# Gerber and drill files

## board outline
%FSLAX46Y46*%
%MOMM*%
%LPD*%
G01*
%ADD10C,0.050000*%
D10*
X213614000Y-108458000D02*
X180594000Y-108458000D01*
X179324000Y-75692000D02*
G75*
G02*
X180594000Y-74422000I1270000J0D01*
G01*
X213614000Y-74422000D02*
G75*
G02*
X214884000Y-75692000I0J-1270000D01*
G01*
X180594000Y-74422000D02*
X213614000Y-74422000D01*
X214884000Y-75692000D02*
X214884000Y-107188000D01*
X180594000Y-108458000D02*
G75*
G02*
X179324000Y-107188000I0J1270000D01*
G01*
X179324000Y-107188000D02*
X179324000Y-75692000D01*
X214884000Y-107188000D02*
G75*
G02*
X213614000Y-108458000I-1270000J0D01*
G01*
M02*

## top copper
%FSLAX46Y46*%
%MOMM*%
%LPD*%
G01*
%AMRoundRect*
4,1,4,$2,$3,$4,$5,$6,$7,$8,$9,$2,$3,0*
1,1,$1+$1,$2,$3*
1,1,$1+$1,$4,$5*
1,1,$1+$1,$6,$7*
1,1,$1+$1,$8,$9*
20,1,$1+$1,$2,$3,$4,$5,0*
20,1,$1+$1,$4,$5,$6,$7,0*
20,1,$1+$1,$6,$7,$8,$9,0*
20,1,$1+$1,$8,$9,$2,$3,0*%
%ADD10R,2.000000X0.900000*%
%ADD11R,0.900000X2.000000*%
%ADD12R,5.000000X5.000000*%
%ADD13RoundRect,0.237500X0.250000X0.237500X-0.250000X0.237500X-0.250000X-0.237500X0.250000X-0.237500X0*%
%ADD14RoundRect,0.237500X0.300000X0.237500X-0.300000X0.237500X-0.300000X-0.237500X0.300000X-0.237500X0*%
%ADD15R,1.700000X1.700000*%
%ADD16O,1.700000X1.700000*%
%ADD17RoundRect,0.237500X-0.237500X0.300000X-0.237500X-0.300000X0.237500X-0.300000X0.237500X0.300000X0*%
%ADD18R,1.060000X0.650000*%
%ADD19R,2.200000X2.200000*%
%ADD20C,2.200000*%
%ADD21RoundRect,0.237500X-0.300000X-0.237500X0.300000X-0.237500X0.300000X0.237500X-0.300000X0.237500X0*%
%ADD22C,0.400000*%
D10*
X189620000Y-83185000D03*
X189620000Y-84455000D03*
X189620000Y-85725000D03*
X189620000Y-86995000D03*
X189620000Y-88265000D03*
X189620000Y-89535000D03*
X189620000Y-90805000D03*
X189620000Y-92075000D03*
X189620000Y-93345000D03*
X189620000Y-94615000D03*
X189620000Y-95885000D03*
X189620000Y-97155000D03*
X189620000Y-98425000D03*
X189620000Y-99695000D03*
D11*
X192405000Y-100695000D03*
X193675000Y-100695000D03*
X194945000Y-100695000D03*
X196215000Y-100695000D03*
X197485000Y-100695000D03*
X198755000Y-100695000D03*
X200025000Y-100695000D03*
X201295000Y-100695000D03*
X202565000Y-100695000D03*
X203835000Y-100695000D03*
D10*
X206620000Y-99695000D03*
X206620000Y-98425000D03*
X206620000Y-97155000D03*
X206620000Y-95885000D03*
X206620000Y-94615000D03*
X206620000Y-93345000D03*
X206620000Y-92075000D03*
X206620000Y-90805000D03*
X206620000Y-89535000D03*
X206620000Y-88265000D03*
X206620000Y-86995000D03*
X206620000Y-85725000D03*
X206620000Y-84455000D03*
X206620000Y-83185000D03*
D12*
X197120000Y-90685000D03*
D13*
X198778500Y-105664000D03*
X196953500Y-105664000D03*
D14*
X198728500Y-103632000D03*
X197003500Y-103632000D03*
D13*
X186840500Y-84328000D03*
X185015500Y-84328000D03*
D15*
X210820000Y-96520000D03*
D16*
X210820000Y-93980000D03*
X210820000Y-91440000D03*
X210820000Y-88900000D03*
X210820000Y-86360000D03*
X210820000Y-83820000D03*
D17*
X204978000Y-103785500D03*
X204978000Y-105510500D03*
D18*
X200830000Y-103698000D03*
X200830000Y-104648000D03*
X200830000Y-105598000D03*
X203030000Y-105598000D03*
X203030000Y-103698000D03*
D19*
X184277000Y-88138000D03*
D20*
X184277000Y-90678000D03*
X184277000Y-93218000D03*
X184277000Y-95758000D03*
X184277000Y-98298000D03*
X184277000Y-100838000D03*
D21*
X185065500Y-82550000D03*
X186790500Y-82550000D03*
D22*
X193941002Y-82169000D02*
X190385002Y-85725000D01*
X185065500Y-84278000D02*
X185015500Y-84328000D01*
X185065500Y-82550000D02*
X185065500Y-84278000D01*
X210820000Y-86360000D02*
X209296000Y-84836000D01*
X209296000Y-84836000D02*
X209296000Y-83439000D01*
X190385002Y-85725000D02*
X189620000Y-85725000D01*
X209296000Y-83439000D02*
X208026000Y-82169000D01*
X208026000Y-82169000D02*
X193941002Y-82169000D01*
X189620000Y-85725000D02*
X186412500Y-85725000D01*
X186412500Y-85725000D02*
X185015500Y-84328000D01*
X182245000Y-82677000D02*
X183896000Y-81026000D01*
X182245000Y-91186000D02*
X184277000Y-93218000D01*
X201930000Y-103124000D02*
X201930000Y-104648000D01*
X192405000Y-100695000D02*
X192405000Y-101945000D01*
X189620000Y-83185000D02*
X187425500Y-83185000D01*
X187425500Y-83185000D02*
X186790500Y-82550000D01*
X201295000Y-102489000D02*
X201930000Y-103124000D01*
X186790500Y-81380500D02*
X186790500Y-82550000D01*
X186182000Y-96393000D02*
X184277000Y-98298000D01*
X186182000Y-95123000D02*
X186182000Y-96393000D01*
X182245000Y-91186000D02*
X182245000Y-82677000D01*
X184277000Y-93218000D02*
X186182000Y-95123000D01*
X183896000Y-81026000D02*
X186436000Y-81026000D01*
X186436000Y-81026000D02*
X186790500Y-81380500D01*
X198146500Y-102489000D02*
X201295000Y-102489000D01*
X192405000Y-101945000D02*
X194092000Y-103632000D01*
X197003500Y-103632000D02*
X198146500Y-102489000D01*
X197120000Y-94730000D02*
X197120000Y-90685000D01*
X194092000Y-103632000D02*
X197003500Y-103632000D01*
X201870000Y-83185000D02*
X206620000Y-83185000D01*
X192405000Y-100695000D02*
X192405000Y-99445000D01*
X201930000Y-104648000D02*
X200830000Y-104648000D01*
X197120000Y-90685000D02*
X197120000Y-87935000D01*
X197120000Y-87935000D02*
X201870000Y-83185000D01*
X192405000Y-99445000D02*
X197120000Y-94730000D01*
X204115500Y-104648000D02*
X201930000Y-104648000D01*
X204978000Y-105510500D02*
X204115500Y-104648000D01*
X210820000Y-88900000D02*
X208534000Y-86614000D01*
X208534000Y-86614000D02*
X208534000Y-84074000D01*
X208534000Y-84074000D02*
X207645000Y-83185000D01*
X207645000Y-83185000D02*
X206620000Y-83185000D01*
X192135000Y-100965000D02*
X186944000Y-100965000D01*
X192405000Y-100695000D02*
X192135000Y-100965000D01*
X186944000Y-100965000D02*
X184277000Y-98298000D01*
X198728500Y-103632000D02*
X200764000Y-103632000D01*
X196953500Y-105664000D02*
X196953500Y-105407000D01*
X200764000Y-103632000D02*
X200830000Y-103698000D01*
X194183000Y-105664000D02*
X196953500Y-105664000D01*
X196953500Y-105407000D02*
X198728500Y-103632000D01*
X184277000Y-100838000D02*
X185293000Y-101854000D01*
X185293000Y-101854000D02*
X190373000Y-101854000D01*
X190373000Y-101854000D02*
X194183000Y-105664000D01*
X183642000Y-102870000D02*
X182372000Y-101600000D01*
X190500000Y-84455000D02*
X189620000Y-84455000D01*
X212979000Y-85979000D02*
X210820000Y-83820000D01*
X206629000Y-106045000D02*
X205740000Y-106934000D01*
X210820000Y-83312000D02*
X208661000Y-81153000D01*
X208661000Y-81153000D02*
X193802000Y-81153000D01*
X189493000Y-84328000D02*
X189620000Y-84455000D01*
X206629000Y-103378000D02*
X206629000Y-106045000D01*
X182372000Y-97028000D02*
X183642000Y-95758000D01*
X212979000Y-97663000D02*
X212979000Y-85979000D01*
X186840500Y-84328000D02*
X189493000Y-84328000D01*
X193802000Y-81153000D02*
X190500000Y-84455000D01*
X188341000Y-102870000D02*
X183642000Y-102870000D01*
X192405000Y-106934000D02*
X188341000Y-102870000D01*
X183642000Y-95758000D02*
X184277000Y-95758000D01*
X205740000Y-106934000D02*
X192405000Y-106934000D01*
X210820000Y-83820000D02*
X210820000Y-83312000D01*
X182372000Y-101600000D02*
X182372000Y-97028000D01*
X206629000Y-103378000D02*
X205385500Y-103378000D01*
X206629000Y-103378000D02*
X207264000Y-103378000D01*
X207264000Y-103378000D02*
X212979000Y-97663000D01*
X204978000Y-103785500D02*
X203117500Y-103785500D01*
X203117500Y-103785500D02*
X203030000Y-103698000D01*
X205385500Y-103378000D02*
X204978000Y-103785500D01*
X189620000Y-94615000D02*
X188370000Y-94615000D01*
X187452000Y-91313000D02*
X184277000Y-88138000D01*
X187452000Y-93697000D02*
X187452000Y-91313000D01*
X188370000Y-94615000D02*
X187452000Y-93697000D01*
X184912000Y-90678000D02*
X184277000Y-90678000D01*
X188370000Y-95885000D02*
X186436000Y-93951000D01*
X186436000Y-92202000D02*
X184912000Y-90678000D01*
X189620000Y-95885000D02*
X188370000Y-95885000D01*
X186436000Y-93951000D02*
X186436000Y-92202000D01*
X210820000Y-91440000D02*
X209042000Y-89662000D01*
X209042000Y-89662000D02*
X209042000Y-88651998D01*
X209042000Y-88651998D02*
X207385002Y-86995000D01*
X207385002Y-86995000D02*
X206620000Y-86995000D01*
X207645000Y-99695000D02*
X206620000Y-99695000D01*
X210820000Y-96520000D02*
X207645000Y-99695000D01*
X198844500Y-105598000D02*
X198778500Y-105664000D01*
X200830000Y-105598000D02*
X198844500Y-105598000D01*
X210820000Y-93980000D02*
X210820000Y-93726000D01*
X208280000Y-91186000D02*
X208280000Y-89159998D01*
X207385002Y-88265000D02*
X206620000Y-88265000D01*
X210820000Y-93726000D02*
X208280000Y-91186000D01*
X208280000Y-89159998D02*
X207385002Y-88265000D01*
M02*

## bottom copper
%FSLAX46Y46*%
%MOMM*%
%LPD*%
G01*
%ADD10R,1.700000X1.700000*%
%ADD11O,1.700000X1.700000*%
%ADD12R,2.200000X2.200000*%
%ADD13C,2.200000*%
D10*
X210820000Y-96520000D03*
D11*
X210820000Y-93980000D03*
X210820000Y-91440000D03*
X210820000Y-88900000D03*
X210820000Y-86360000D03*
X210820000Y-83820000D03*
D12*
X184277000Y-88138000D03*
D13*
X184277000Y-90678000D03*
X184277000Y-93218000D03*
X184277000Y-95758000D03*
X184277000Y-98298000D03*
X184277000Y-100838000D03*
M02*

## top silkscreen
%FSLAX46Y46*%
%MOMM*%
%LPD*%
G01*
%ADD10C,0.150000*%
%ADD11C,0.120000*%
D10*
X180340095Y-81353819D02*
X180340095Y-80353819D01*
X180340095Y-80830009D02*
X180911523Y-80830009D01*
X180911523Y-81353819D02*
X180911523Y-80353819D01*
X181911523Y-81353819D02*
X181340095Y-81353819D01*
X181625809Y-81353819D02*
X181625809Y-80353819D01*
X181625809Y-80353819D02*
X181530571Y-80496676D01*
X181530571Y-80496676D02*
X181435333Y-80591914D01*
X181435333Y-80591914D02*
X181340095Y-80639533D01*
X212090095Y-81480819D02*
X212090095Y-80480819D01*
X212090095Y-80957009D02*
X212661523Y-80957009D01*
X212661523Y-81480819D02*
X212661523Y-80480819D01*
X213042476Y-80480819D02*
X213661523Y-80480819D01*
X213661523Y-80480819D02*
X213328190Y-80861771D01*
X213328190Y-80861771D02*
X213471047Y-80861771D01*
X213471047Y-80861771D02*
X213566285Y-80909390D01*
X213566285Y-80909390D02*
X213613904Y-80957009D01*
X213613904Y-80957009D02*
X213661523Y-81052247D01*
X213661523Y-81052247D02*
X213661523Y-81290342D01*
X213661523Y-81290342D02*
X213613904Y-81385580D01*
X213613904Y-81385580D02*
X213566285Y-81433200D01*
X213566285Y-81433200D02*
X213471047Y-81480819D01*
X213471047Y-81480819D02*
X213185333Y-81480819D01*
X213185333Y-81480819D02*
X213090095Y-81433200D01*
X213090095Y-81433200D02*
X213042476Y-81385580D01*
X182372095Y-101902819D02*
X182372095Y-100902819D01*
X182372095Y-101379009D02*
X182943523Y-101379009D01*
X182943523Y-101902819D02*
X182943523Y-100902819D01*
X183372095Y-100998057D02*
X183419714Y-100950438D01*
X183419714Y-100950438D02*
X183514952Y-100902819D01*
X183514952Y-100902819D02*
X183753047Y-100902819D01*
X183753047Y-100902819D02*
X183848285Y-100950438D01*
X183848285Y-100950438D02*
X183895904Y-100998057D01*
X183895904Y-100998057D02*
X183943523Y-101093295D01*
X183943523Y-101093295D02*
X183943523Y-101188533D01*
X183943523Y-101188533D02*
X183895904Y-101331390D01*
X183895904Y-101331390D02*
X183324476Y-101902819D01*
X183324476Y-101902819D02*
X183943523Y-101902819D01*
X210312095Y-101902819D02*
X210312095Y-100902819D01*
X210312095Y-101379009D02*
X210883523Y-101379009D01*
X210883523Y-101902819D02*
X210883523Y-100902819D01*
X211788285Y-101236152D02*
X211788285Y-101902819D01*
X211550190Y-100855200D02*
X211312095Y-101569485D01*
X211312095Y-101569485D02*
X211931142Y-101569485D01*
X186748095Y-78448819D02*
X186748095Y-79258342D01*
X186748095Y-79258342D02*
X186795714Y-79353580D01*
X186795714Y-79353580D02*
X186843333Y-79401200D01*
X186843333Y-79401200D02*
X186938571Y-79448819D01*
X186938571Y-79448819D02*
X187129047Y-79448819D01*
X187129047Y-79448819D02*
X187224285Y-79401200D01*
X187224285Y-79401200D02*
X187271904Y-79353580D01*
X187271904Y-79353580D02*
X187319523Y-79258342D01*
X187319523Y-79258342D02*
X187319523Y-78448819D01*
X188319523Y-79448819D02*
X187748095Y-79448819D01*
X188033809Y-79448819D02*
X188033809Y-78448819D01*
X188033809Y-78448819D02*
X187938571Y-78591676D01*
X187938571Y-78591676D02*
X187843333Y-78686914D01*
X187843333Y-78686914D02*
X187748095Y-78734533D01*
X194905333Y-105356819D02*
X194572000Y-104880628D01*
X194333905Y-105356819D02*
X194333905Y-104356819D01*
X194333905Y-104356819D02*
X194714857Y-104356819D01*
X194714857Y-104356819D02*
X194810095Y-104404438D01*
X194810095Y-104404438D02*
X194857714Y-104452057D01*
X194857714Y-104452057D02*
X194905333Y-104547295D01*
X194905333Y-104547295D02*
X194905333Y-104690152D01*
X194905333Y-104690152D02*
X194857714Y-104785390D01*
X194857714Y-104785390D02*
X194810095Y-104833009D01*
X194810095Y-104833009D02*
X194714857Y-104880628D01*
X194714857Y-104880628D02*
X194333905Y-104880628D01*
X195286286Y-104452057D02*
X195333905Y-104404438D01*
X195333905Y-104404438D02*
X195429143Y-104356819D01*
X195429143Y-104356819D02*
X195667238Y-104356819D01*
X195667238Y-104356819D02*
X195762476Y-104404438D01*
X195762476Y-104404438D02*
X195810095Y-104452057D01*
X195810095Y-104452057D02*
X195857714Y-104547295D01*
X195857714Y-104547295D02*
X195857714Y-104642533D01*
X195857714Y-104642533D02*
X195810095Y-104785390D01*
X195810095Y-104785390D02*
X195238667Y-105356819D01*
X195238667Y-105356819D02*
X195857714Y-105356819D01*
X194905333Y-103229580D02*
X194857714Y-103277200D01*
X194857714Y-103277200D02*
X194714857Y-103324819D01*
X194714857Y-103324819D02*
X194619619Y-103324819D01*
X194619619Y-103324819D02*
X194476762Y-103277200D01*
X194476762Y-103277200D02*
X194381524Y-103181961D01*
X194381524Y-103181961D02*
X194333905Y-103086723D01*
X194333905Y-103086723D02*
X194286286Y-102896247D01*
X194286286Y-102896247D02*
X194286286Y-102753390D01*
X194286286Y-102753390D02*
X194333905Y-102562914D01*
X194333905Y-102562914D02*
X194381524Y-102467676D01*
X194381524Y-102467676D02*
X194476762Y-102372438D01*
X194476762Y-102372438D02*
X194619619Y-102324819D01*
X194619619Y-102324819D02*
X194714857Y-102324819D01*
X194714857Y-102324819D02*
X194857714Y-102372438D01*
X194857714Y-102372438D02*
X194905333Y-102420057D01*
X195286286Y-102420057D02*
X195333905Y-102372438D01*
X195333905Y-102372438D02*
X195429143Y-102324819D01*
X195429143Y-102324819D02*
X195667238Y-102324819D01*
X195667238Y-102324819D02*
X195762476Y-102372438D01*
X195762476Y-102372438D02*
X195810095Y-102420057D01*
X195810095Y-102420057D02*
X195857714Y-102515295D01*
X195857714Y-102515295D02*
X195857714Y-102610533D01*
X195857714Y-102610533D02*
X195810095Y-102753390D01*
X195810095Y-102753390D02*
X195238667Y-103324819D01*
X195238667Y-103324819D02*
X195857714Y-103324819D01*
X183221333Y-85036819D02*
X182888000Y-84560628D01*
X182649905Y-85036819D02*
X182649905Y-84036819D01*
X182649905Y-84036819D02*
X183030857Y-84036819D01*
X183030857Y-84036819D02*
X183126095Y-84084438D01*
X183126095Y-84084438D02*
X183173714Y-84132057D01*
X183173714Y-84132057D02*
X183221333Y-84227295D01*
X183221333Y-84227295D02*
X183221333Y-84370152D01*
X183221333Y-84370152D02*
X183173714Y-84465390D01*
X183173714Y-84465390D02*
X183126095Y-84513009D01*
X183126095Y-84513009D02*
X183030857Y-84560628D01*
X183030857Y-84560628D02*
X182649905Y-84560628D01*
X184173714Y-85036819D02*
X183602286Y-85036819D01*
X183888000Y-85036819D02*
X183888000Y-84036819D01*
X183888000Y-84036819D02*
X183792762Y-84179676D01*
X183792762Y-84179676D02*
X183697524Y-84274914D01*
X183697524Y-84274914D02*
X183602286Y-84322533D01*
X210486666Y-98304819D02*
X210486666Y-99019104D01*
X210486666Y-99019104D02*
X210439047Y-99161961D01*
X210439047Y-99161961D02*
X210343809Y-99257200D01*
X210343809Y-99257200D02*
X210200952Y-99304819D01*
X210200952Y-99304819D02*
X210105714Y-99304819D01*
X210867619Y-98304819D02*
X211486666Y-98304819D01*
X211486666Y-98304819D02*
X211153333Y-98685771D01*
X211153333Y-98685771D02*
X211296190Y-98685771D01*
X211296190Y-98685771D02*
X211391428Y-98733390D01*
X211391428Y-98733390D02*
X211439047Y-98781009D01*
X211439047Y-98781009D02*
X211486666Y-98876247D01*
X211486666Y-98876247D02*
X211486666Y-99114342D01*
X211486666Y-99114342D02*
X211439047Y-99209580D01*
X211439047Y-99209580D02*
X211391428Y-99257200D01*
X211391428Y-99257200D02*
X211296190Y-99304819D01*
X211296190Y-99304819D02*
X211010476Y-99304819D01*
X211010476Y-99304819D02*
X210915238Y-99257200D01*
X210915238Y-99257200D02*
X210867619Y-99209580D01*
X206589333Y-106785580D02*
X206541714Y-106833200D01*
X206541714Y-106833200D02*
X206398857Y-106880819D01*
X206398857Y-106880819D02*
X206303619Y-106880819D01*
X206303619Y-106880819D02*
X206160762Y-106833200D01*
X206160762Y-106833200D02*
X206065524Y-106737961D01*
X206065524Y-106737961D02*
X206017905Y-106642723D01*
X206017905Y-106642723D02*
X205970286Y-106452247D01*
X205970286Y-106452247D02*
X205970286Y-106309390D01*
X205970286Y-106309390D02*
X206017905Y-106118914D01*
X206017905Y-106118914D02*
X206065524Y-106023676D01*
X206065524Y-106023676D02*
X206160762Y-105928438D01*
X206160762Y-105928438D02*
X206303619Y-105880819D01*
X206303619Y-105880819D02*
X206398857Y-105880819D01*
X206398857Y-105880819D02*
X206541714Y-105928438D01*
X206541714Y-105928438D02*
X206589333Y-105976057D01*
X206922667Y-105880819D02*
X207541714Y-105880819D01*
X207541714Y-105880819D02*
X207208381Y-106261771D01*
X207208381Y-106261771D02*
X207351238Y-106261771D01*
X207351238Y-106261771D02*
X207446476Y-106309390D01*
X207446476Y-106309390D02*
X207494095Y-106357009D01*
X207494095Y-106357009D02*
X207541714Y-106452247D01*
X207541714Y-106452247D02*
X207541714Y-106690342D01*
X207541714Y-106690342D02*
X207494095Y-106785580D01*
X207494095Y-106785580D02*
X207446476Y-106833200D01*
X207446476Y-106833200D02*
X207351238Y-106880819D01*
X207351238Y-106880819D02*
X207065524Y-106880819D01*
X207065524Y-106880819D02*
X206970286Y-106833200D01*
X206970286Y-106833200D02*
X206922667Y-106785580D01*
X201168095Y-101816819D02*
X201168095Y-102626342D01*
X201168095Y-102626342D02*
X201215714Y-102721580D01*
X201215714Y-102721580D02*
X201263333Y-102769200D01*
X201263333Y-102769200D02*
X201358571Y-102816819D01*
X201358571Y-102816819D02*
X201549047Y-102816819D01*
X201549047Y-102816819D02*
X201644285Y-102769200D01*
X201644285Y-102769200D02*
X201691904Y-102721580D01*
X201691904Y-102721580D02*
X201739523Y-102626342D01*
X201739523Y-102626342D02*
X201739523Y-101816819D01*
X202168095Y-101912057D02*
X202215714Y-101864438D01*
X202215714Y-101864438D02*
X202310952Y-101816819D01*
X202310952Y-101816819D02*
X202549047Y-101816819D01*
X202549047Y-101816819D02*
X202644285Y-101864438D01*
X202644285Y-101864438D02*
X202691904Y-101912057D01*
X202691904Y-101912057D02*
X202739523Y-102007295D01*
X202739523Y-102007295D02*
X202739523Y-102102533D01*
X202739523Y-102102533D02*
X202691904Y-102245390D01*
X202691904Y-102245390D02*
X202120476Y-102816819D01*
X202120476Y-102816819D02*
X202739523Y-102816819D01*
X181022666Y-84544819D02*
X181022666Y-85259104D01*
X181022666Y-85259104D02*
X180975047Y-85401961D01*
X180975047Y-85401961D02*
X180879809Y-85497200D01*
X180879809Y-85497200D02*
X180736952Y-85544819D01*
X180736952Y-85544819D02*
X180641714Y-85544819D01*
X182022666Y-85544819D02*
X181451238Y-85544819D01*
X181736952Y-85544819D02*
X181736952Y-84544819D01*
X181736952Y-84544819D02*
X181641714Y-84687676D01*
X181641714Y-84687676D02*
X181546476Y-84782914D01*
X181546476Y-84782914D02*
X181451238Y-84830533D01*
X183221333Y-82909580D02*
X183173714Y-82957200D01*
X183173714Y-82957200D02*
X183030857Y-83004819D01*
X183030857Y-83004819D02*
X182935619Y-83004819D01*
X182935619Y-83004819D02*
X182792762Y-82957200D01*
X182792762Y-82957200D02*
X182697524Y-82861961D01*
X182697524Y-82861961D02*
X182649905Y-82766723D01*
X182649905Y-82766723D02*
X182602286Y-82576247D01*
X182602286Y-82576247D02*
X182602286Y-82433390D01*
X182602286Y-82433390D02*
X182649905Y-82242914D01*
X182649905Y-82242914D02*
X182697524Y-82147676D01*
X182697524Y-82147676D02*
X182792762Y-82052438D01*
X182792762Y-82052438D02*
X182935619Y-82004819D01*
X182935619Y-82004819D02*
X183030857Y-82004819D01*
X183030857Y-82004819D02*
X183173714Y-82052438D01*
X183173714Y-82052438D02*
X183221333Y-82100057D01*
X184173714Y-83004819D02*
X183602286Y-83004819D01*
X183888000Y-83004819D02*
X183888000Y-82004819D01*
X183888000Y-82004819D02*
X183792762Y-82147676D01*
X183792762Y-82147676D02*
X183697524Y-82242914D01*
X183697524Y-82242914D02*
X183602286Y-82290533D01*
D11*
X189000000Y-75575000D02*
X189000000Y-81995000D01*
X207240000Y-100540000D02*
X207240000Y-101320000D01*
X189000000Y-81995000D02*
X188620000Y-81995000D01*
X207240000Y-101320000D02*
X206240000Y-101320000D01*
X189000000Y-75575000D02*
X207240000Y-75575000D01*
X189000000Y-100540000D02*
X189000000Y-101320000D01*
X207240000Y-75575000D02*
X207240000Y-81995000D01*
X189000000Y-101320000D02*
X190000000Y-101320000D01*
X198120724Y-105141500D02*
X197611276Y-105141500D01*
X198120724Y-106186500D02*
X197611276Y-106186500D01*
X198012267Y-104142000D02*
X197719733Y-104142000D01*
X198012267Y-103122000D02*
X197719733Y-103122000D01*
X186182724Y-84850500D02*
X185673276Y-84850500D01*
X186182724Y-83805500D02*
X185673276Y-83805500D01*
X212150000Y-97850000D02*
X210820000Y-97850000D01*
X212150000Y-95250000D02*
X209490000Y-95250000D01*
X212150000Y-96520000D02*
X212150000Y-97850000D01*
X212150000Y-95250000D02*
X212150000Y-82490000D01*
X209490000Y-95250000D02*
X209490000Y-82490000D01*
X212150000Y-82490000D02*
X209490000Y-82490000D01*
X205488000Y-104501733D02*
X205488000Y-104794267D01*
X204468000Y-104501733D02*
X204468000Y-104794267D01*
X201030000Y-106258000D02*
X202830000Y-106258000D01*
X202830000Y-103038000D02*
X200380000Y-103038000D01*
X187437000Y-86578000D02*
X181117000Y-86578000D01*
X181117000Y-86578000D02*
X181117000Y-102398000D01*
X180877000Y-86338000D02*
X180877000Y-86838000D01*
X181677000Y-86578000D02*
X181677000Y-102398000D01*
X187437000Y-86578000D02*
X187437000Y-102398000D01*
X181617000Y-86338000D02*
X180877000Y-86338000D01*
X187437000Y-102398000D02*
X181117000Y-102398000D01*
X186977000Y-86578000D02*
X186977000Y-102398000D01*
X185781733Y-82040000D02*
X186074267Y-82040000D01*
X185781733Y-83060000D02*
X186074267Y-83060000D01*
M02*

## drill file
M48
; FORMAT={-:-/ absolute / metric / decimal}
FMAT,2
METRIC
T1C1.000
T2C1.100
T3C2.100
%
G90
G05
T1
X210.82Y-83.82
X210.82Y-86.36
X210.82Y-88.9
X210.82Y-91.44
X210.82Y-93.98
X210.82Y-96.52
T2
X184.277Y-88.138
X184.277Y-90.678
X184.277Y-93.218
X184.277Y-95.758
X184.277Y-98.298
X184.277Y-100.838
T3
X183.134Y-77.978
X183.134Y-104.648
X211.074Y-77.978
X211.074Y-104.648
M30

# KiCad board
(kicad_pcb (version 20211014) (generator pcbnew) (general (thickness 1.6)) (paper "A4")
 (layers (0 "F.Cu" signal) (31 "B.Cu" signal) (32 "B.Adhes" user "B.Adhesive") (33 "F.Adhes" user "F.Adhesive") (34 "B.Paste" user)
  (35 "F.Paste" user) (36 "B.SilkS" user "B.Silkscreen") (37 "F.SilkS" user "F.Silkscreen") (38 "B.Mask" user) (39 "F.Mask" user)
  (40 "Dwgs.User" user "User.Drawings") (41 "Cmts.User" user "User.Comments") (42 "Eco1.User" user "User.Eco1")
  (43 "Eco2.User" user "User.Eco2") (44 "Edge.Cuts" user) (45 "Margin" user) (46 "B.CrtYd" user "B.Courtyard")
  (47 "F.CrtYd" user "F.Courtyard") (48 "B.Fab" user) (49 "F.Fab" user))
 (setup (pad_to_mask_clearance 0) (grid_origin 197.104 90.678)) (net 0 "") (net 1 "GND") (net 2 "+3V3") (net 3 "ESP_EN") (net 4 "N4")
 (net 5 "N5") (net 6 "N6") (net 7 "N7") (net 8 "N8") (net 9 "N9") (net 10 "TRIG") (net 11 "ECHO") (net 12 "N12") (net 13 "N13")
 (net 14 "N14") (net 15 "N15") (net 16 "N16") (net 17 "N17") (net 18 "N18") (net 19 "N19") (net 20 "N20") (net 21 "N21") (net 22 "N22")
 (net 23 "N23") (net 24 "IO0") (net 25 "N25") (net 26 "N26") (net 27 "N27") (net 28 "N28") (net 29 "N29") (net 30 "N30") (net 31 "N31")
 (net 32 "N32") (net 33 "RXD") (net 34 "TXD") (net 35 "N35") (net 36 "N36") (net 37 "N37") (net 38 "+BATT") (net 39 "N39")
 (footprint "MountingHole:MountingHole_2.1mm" (layer "F.Cu") (at 183.134 77.978)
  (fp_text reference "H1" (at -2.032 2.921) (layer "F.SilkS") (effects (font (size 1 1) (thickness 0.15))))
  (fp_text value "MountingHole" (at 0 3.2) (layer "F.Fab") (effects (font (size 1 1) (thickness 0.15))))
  (pad "" np_thru_hole circle locked (at 0 0) (size 2.1 2.1) (drill 2.1) (layers *.Cu *.Mask)))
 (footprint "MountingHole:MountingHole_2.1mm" (layer "F.Cu") (at 211.074 77.978)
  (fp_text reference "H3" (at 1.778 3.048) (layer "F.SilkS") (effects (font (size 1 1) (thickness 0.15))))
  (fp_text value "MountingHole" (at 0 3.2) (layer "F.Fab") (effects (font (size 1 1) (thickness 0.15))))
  (pad "" np_thru_hole circle locked (at 0 0) (size 2.1 2.1) (drill 2.1) (layers *.Cu *.Mask)))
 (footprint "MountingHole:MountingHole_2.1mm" (layer "F.Cu") (at 183.134 104.648)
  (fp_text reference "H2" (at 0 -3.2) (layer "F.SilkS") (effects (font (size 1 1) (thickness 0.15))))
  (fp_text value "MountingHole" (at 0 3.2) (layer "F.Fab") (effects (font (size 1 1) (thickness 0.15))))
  (pad "" np_thru_hole circle locked (at 0 0) (size 2.1 2.1) (drill 2.1) (layers *.Cu *.Mask)))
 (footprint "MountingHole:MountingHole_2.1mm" (layer "F.Cu") (at 211.074 104.648)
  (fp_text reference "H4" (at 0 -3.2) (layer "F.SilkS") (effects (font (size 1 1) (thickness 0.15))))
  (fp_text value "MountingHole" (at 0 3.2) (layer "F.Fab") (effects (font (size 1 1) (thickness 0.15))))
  (pad "" np_thru_hole circle locked (at 0 0) (size 2.1 2.1) (drill 2.1) (layers *.Cu *.Mask)))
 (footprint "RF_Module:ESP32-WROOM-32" (layer "F.Cu") (at 198.12 91.44)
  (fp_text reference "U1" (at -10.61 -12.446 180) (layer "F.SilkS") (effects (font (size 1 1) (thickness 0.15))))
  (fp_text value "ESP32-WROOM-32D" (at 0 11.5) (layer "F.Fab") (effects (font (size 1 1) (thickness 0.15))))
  (fp_line (start -9.12 -15.865) (end -9.12 -9.445) (layer "F.SilkS") (width 0.12))
  (fp_line (start 9.12 9.1) (end 9.12 9.88) (layer "F.SilkS") (width 0.12))
  (fp_line (start -9.12 -9.445) (end -9.5 -9.445) (layer "F.SilkS") (width 0.12))
  (fp_line (start 9.12 9.88) (end 8.12 9.88) (layer "F.SilkS") (width 0.12))
  (fp_line (start -9.12 -15.865) (end 9.12 -15.865) (layer "F.SilkS") (width 0.12))
  (fp_line (start -9.12 9.1) (end -9.12 9.88) (layer "F.SilkS") (width 0.12))
  (fp_line (start 9.12 -15.865) (end 9.12 -9.445) (layer "F.SilkS") (width 0.12))
  (fp_line (start -9.12 9.88) (end -8.12 9.88) (layer "F.SilkS") (width 0.12))
  (pad "1" smd rect locked (at -8.5 -8.255) (size 2 0.9) (layers "F.Cu" "F.Paste" "F.Mask") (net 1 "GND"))
  (pad "2" smd rect locked (at -8.5 -6.985) (size 2 0.9) (layers "F.Cu" "F.Paste" "F.Mask") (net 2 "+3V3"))
  (pad "3" smd rect locked (at -8.5 -5.715) (size 2 0.9) (layers "F.Cu" "F.Paste" "F.Mask") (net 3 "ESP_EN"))
  (pad "4" smd rect locked (at -8.5 -4.445) (size 2 0.9) (layers "F.Cu" "F.Paste" "F.Mask") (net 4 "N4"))
  (pad "5" smd rect locked (at -8.5 -3.175) (size 2 0.9) (layers "F.Cu" "F.Paste" "F.Mask") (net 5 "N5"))
  (pad "6" smd rect locked (at -8.5 -1.905) (size 2 0.9) (layers "F.Cu" "F.Paste" "F.Mask") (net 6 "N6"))
  (pad "7" smd rect locked (at -8.5 -0.635) (size 2 0.9) (layers "F.Cu" "F.Paste" "F.Mask") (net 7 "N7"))
  (pad "8" smd rect locked (at -8.5 0.635) (size 2 0.9) (layers "F.Cu" "F.Paste" "F.Mask") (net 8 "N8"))
  (pad "9" smd rect locked (at -8.5 1.905) (size 2 0.9) (layers "F.Cu" "F.Paste" "F.Mask") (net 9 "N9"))
  (pad "10" smd rect locked (at -8.5 3.175) (size 2 0.9) (layers "F.Cu" "F.Paste" "F.Mask") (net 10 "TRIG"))
  (pad "11" smd rect locked (at -8.5 4.445) (size 2 0.9) (layers "F.Cu" "F.Paste" "F.Mask") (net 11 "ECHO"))
  (pad "12" smd rect locked (at -8.5 5.715) (size 2 0.9) (layers "F.Cu" "F.Paste" "F.Mask") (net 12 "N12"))
  (pad "13" smd rect locked (at -8.5 6.985) (size 2 0.9) (layers "F.Cu" "F.Paste" "F.Mask") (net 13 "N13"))
  (pad "14" smd rect locked (at -8.5 8.255) (size 2 0.9) (layers "F.Cu" "F.Paste" "F.Mask") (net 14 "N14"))
  (pad "15" smd rect locked (at -5.715 9.255 90) (size 2 0.9) (layers "F.Cu" "F.Paste" "F.Mask") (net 1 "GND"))
  (pad "16" smd rect locked (at -4.445 9.255 90) (size 2 0.9) (layers "F.Cu" "F.Paste" "F.Mask") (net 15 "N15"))
  (pad "17" smd rect locked (at -3.175 9.255 90) (size 2 0.9) (layers "F.Cu" "F.Paste" "F.Mask") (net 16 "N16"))
  (pad "18" smd rect locked (at -1.905 9.255 90) (size 2 0.9) (layers "F.Cu" "F.Paste" "F.Mask") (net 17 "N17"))
  (pad "19" smd rect locked (at -0.635 9.255 90) (size 2 0.9) (layers "F.Cu" "F.Paste" "F.Mask") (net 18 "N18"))
  (pad "20" smd rect locked (at 0.635 9.255 90) (size 2 0.9) (layers "F.Cu" "F.Paste" "F.Mask") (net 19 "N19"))
  (pad "21" smd rect locked (at 1.905 9.255 90) (size 2 0.9) (layers "F.Cu" "F.Paste" "F.Mask") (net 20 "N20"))
  (pad "22" smd rect locked (at 3.175 9.255 90) (size 2 0.9) (layers "F.Cu" "F.Paste" "F.Mask") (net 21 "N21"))
  (pad "23" smd rect locked (at 4.445 9.255 90) (size 2 0.9) (layers "F.Cu" "F.Paste" "F.Mask") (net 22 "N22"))
  (pad "24" smd rect locked (at 5.715 9.255 90) (size 2 0.9) (layers "F.Cu" "F.Paste" "F.Mask") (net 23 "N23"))
  (pad "25" smd rect locked (at 8.5 8.255) (size 2 0.9) (layers "F.Cu" "F.Paste" "F.Mask") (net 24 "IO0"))
  (pad "26" smd rect locked (at 8.5 6.985) (size 2 0.9) (layers "F.Cu" "F.Paste" "F.Mask") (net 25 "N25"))
  (pad "27" smd rect locked (at 8.5 5.715) (size 2 0.9) (layers "F.Cu" "F.Paste" "F.Mask") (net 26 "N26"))
  (pad "28" smd rect locked (at 8.5 4.445) (size 2 0.9) (layers "F.Cu" "F.Paste" "F.Mask") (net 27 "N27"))
  (pad "29" smd rect locked (at 8.5 3.175) (size 2 0.9) (layers "F.Cu" "F.Paste" "F.Mask") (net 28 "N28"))
  (pad "30" smd rect locked (at 8.5 1.905) (size 2 0.9) (layers "F.Cu" "F.Paste" "F.Mask") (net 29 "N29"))
  (pad "31" smd rect locked (at 8.5 0.635) (size 2 0.9) (layers "F.Cu" "F.Paste" "F.Mask") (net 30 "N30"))
  (pad "32" smd rect locked (at 8.5 -0.635) (size 2 0.9) (layers "F.Cu" "F.Paste" "F.Mask") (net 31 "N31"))
  (pad "33" smd rect locked (at 8.5 -1.905) (size 2 0.9) (layers "F.Cu" "F.Paste" "F.Mask") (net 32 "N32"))
  (pad "34" smd rect locked (at 8.5 -3.175) (size 2 0.9) (layers "F.Cu" "F.Paste" "F.Mask") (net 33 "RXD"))
  (pad "35" smd rect locked (at 8.5 -4.445) (size 2 0.9) (layers "F.Cu" "F.Paste" "F.Mask") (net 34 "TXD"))
  (pad "36" smd rect locked (at 8.5 -5.715) (size 2 0.9) (layers "F.Cu" "F.Paste" "F.Mask") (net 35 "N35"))
  (pad "37" smd rect locked (at 8.5 -6.985) (size 2 0.9) (layers "F.Cu" "F.Paste" "F.Mask") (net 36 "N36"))
  (pad "38" smd rect locked (at 8.5 -8.255) (size 2 0.9) (layers "F.Cu" "F.Paste" "F.Mask") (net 1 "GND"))
  (pad "39" smd rect locked (at -1 -0.755) (size 5 5) (layers "F.Cu" "F.Paste" "F.Mask") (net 1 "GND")))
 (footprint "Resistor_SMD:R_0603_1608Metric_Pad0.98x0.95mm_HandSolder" (layer "F.Cu") (at 197.866 105.664 180)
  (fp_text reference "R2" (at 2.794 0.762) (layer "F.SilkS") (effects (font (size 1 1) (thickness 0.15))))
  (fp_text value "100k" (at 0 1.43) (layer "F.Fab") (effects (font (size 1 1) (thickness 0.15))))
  (fp_line (start -0.254724 0.5225) (end 0.254724 0.5225) (layer "F.SilkS") (width 0.12))
  (fp_line (start -0.254724 -0.5225) (end 0.254724 -0.5225) (layer "F.SilkS") (width 0.12))
  (pad "1" smd roundrect locked (at -0.9125 0 180) (size 0.975 0.95) (layers "F.Cu" "F.Paste" "F.Mask") (roundrect_rratio 0.25)
   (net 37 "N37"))
  (pad "2" smd roundrect locked (at 0.9125 0 180) (size 0.975 0.95) (layers "F.Cu" "F.Paste" "F.Mask") (roundrect_rratio 0.25)
   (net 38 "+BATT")))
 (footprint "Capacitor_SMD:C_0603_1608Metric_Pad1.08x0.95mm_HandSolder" (layer "F.Cu") (at 197.866 103.632 180)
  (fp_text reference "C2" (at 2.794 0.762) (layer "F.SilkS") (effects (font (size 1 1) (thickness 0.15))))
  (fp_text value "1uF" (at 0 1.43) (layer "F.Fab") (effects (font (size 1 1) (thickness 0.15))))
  (fp_line (start -0.146267 -0.51) (end 0.146267 -0.51) (layer "F.SilkS") (width 0.12))
  (fp_line (start -0.146267 0.51) (end 0.146267 0.51) (layer "F.SilkS") (width 0.12))
  (pad "1" smd roundrect locked (at -0.8625 0 180) (size 1.075 0.95) (layers "F.Cu" "F.Paste" "F.Mask") (roundrect_rratio 0.25)
   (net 38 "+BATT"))
  (pad "2" smd roundrect locked (at 0.8625 0 180) (size 1.075 0.95) (layers "F.Cu" "F.Paste" "F.Mask") (roundrect_rratio 0.25) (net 1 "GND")))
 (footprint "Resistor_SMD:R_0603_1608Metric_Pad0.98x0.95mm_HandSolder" (layer "F.Cu") (at 185.928 84.328 180)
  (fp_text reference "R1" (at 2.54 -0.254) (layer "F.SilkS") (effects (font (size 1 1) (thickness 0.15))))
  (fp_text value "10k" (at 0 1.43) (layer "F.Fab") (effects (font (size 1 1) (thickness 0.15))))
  (fp_line (start -0.254724 -0.5225) (end 0.254724 -0.5225) (layer "F.SilkS") (width 0.12))
  (fp_line (start -0.254724 0.5225) (end 0.254724 0.5225) (layer "F.SilkS") (width 0.12))
  (pad "1" smd roundrect locked (at -0.9125 0 180) (size 0.975 0.95) (layers "F.Cu" "F.Paste" "F.Mask") (roundrect_rratio 0.25)
   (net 2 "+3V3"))
  (pad "2" smd roundrect locked (at 0.9125 0 180) (size 0.975 0.95) (layers "F.Cu" "F.Paste" "F.Mask") (roundrect_rratio 0.25)
   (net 3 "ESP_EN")))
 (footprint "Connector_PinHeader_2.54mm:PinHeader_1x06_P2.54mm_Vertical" (layer "F.Cu") (at 210.82 96.52 180)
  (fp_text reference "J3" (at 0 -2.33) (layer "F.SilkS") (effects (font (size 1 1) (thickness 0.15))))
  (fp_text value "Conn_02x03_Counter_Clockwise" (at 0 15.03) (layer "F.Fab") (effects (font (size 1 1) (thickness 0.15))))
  (fp_line (start -1.33 -1.33) (end 0 -1.33) (layer "F.SilkS") (width 0.12))
  (fp_line (start -1.33 1.27) (end 1.33 1.27) (layer "F.SilkS") (width 0.12))
  (fp_line (start -1.33 0) (end -1.33 -1.33) (layer "F.SilkS") (width 0.12))
  (fp_line (start -1.33 1.27) (end -1.33 14.03) (layer "F.SilkS") (width 0.12))
  (fp_line (start 1.33 1.27) (end 1.33 14.03) (layer "F.SilkS") (width 0.12))
  (fp_line (start -1.33 14.03) (end 1.33 14.03) (layer "F.SilkS") (width 0.12))
  (pad "1" thru_hole rect locked (at 0 0 180) (size 1.7 1.7) (drill 1) (layers *.Cu *.Mask) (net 24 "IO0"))
  (pad "2" thru_hole oval locked (at 0 2.54 180) (size 1.7 1.7) (drill 1) (layers *.Cu *.Mask) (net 33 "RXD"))
  (pad "3" thru_hole oval locked (at 0 5.08 180) (size 1.7 1.7) (drill 1) (layers *.Cu *.Mask) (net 34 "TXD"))
  (pad "4" thru_hole oval locked (at 0 7.62 180) (size 1.7 1.7) (drill 1) (layers *.Cu *.Mask) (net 1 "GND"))
  (pad "5" thru_hole oval locked (at 0 10.16 180) (size 1.7 1.7) (drill 1) (layers *.Cu *.Mask) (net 3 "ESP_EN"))
  (pad "6" thru_hole oval locked (at 0 12.7 180) (size 1.7 1.7) (drill 1) (layers *.Cu *.Mask) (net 2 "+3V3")))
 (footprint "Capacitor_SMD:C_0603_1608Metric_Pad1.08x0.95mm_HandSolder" (layer "F.Cu") (at 204.978 104.648 -90)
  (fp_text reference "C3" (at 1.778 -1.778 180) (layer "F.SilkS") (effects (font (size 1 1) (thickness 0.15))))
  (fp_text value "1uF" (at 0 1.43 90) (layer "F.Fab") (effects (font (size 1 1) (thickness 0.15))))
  (fp_line (start -0.146267 -0.51) (end 0.146267 -0.51) (layer "F.SilkS") (width 0.12))
  (fp_line (start -0.146267 0.51) (end 0.146267 0.51) (layer "F.SilkS") (width 0.12))
  (pad "1" smd roundrect locked (at -0.8625 0 270) (size 1.075 0.95) (layers "F.Cu" "F.Paste" "F.Mask") (roundrect_rratio 0.25)
   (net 2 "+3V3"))
  (pad "2" smd roundrect locked (at 0.8625 0 270) (size 1.075 0.95) (layers "F.Cu" "F.Paste" "F.Mask") (roundrect_rratio 0.25) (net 1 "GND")))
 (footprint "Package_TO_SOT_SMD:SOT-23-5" (layer "F.Cu") (at 201.93 104.648)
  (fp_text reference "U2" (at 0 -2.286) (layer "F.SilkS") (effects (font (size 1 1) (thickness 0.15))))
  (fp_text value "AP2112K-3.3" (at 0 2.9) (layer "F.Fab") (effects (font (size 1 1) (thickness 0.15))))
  (fp_line (start -0.9 1.61) (end 0.9 1.61) (layer "F.SilkS") (width 0.12))
  (fp_line (start 0.9 -1.61) (end -1.55 -1.61) (layer "F.SilkS") (width 0.12))
  (pad "1" smd rect locked (at -1.1 -0.95) (size 1.06 0.65) (layers "F.Cu" "F.Paste" "F.Mask") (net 38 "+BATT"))
  (pad "2" smd rect locked (at -1.1 0) (size 1.06 0.65) (layers "F.Cu" "F.Paste" "F.Mask") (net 1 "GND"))
  (pad "3" smd rect locked (at -1.1 0.95) (size 1.06 0.65) (layers "F.Cu" "F.Paste" "F.Mask") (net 37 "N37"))
  (pad "4" smd rect locked (at 1.1 0.95) (size 1.06 0.65) (layers "F.Cu" "F.Paste" "F.Mask") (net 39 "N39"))
  (pad "5" smd rect locked (at 1.1 -0.95) (size 1.06 0.65) (layers "F.Cu" "F.Paste" "F.Mask") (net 2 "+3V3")))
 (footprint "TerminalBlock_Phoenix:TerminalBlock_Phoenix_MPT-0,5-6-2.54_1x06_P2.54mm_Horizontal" (layer "F.Cu") (at 184.277 88.138 -90)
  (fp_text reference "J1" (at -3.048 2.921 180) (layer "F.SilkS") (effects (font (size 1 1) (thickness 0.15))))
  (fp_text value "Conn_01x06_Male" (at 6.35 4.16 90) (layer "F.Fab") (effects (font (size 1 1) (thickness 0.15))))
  (fp_line (start -1.56 -3.16) (end -1.56 3.16) (layer "F.SilkS") (width 0.12))
  (fp_line (start -1.56 3.16) (end 14.26 3.16) (layer "F.SilkS") (width 0.12))
  (fp_line (start -1.8 3.4) (end -1.3 3.4) (layer "F.SilkS") (width 0.12))
  (fp_line (start -1.56 2.6) (end 14.26 2.6) (layer "F.SilkS") (width 0.12))
  (fp_line (start -1.56 -3.16) (end 14.26 -3.16) (layer "F.SilkS") (width 0.12))
  (fp_line (start -1.8 2.66) (end -1.8 3.4) (layer "F.SilkS") (width 0.12))
  (fp_line (start 14.26 -3.16) (end 14.26 3.16) (layer "F.SilkS") (width 0.12))
  (fp_line (start -1.56 -2.7) (end 14.26 -2.7) (layer "F.SilkS") (width 0.12))
  (pad "1" thru_hole rect locked (at 0 0 270) (size 2.2 2.2) (drill 1.1) (layers *.Cu *.Mask) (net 10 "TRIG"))
  (pad "2" thru_hole circle locked (at 2.54 0 270) (size 2.2 2.2) (drill 1.1) (layers *.Cu *.Mask) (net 11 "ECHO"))
  (pad "3" thru_hole circle locked (at 5.08 0 270) (size 2.2 2.2) (drill 1.1) (layers *.Cu *.Mask) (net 1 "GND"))
  (pad "4" thru_hole circle locked (at 7.62 0 270) (size 2.2 2.2) (drill 1.1) (layers *.Cu *.Mask) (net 2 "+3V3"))
  (pad "5" thru_hole circle locked (at 10.16 0 270) (size 2.2 2.2) (drill 1.1) (layers *.Cu *.Mask) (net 1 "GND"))
  (pad "6" thru_hole circle locked (at 12.7 0 270) (size 2.2 2.2) (drill 1.1) (layers *.Cu *.Mask) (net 38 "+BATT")))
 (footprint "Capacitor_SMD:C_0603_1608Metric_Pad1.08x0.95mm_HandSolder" (layer "F.Cu") (at 185.928 82.55)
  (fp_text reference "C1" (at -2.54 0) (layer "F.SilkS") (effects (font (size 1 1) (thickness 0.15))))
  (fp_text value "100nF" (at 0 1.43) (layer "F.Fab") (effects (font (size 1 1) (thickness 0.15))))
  (fp_line (start -0.146267 -0.51) (end 0.146267 -0.51) (layer "F.SilkS") (width 0.12))
  (fp_line (start -0.146267 0.51) (end 0.146267 0.51) (layer "F.SilkS") (width 0.12))
  (pad "1" smd roundrect locked (at -0.8625 0) (size 1.075 0.95) (layers "F.Cu" "F.Paste" "F.Mask") (roundrect_rratio 0.25) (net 3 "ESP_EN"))
  (pad "2" smd roundrect locked (at 0.8625 0) (size 1.075 0.95) (layers "F.Cu" "F.Paste" "F.Mask") (roundrect_rratio 0.25) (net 1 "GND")))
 (gr_line (start 213.614 108.458) (end 180.594 108.458) (layer "Edge.Cuts") (width 0.05))
 (gr_arc (start 179.324 75.692) (mid 179.695974 74.793974) (end 180.594 74.422) (layer "Edge.Cuts") (width 0.05))
 (gr_arc (start 213.614 74.422) (mid 214.512026 74.793974) (end 214.884 75.692) (layer "Edge.Cuts") (width 0.05))
 (gr_line (start 180.594 74.422) (end 213.614 74.422) (layer "Edge.Cuts") (width 0.05))
 (gr_line (start 214.884 75.692) (end 214.884 107.188) (layer "Edge.Cuts") (width 0.05))
 (gr_arc (start 180.594 108.458) (mid 179.695974 108.086026) (end 179.324 107.188) (layer "Edge.Cuts") (width 0.05))
 (gr_line (start 179.324 107.188) (end 179.324 75.692) (layer "Edge.Cuts") (width 0.05))
 (gr_arc (start 214.884 107.188) (mid 214.512026 108.086026) (end 213.614 108.458) (layer "Edge.Cuts") (width 0.05))
 (segment (start 193.941002 82.169) (end 190.385002 85.725) (width 0.4) (layer "F.Cu") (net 3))
 (segment (start 185.0655 84.278) (end 185.0155 84.328) (width 0.4) (layer "F.Cu") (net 3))
 (segment (start 185.0655 82.55) (end 185.0655 84.278) (width 0.4) (layer "F.Cu") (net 3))
 (segment (start 210.82 86.36) (end 209.296 84.836) (width 0.4) (layer "F.Cu") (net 3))
 (segment (start 209.296 84.836) (end 209.296 83.439) (width 0.4) (layer "F.Cu") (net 3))
 (segment (start 190.385002 85.725) (end 189.62 85.725) (width 0.4) (layer "F.Cu") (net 3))
 (segment (start 209.296 83.439) (end 208.026 82.169) (width 0.4) (layer "F.Cu") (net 3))
 (segment (start 208.026 82.169) (end 193.941002 82.169) (width 0.4) (layer "F.Cu") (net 3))
 (segment (start 189.62 85.725) (end 186.4125 85.725) (width 0.4) (layer "F.Cu") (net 3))
 (segment (start 186.4125 85.725) (end 185.0155 84.328) (width 0.4) (layer "F.Cu") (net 3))
 (segment (start 182.245 82.677) (end 183.896 81.026) (width 0.4) (layer "F.Cu") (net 1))
 (segment (start 182.245 91.186) (end 184.277 93.218) (width 0.4) (layer "F.Cu") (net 1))
 (segment (start 201.93 103.124) (end 201.93 104.648) (width 0.4) (layer "F.Cu") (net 1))
 (segment (start 192.405 100.695) (end 192.405 101.945) (width 0.4) (layer "F.Cu") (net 1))
 (segment (start 189.62 83.185) (end 187.4255 83.185) (width 0.4) (layer "F.Cu") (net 1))
 (segment (start 187.4255 83.185) (end 186.7905 82.55) (width 0.4) (layer "F.Cu") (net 1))
 (segment (start 201.295 102.489) (end 201.93 103.124) (width 0.4) (layer "F.Cu") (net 1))
 (segment (start 186.7905 81.3805) (end 186.7905 82.55) (width 0.4) (layer "F.Cu") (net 1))
 (segment (start 186.182 96.393) (end 184.277 98.298) (width 0.4) (layer "F.Cu") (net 1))
 (segment (start 186.182 95.123) (end 186.182 96.393) (width 0.4) (layer "F.Cu") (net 1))
 (segment (start 182.245 91.186) (end 182.245 82.677) (width 0.4) (layer "F.Cu") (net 1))
 (segment (start 184.277 93.218) (end 186.182 95.123) (width 0.4) (layer "F.Cu") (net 1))
 (segment (start 183.896 81.026) (end 186.436 81.026) (width 0.4) (layer "F.Cu") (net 1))
 (segment (start 186.436 81.026) (end 186.7905 81.3805) (width 0.4) (layer "F.Cu") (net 1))
 (segment (start 198.1465 102.489) (end 201.295 102.489) (width 0.4) (layer "F.Cu") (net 1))
 (segment (start 192.405 101.945) (end 194.092 103.632) (width 0.4) (layer "F.Cu") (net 1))
 (segment (start 197.0035 103.632) (end 198.1465 102.489) (width 0.4) (layer "F.Cu") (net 1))
 (segment (start 197.12 94.73) (end 197.12 90.685) (width 0.4) (layer "F.Cu") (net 1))
 (segment (start 194.092 103.632) (end 197.0035 103.632) (width 0.4) (layer "F.Cu") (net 1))
 (segment (start 201.87 83.185) (end 206.62 83.185) (width 0.4) (layer "F.Cu") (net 1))
 (segment (start 192.405 100.695) (end 192.405 99.445) (width 0.4) (layer "F.Cu") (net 1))
 (segment (start 201.93 104.648) (end 200.83 104.648) (width 0.4) (layer "F.Cu") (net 1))
 (segment (start 197.12 90.685) (end 197.12 87.935) (width 0.4) (layer "F.Cu") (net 1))
 (segment (start 197.12 87.935) (end 201.87 83.185) (width 0.4) (layer "F.Cu") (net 1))
 (segment (start 192.405 99.445) (end 197.12 94.73) (width 0.4) (layer "F.Cu") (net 1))
 (segment (start 204.1155 104.648) (end 201.93 104.648) (width 0.4) (layer "F.Cu") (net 1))
 (segment (start 204.978 105.5105) (end 204.1155 104.648) (width 0.4) (layer "F.Cu") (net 1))
 (segment (start 210.82 88.9) (end 208.534 86.614) (width 0.4) (layer "F.Cu") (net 1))
 (segment (start 208.534 86.614) (end 208.534 84.074) (width 0.4) (layer "F.Cu") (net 1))
 (segment (start 208.534 84.074) (end 207.645 83.185) (width 0.4) (layer "F.Cu") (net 1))
 (segment (start 207.645 83.185) (end 206.62 83.185) (width 0.4) (layer "F.Cu") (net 1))
 (segment (start 192.135 100.965) (end 186.944 100.965) (width 0.4) (layer "F.Cu") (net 1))
 (segment (start 192.405 100.695) (end 192.135 100.965) (width 0.4) (layer "F.Cu") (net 1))
 (segment (start 186.944 100.965) (end 184.277 98.298) (width 0.4) (layer "F.Cu") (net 1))
 (segment (start 198.7285 103.632) (end 200.764 103.632) (width 0.4) (layer "F.Cu") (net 38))
 (segment (start 196.9535 105.664) (end 196.9535 105.407) (width 0.4) (layer "F.Cu") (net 38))
 (segment (start 200.764 103.632) (end 200.83 103.698) (width 0.4) (layer "F.Cu") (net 38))
 (segment (start 194.183 105.664) (end 196.9535 105.664) (width 0.4) (layer "F.Cu") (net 38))
 (segment (start 196.9535 105.407) (end 198.7285 103.632) (width 0.4) (layer "F.Cu") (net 38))
 (segment (start 184.277 100.838) (end 185.293 101.854) (width 0.4) (layer "F.Cu") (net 38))
 (segment (start 185.293 101.854) (end 190.373 101.854) (width 0.4) (layer "F.Cu") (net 38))
 (segment (start 190.373 101.854) (end 194.183 105.664) (width 0.4) (layer "F.Cu") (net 38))
 (segment (start 183.642 102.87) (end 182.372 101.6) (width 0.4) (layer "F.Cu") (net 2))
 (segment (start 190.5 84.455) (end 189.62 84.455) (width 0.4) (layer "F.Cu") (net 2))
 (segment (start 212.979 85.979) (end 210.82 83.82) (width 0.4) (layer "F.Cu") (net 2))
 (segment (start 206.629 106.045) (end 205.74 106.934) (width 0.4) (layer "F.Cu") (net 2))
 (segment (start 210.82 83.312) (end 208.661 81.153) (width 0.4) (layer "F.Cu") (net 2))
 (segment (start 208.661 81.153) (end 193.802 81.153) (width 0.4) (layer "F.Cu") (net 2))
 (segment (start 189.493 84.328) (end 189.62 84.455) (width 0.4) (layer "F.Cu") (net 2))
 (segment (start 206.629 103.378) (end 206.629 106.045) (width 0.4) (layer "F.Cu") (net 2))
 (segment (start 182.372 97.028) (end 183.642 95.758) (width 0.4) (layer "F.Cu") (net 2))
 (segment (start 212.979 97.663) (end 212.979 85.979) (width 0.4) (layer "F.Cu") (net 2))
 (segment (start 186.8405 84.328) (end 189.493 84.328) (width 0.4) (layer "F.Cu") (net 2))
 (segment (start 193.802 81.153) (end 190.5 84.455) (width 0.4) (layer "F.Cu") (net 2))
 (segment (start 188.341 102.87) (end 183.642 102.87) (width 0.4) (layer "F.Cu") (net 2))
 (segment (start 192.405 106.934) (end 188.341 102.87) (width 0.4) (layer "F.Cu") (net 2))
 (segment (start 183.642 95.758) (end 184.277 95.758) (width 0.4) (layer "F.Cu") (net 2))
 (segment (start 205.74 106.934) (end 192.405 106.934) (width 0.4) (layer "F.Cu") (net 2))
 (segment (start 210.82 83.82) (end 210.82 83.312) (width 0.4) (layer "F.Cu") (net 2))
 (segment (start 182.372 101.6) (end 182.372 97.028) (width 0.4) (layer "F.Cu") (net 2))
 (segment (start 206.629 103.378) (end 205.3855 103.378) (width 0.4) (layer "F.Cu") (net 2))
 (segment (start 206.629 103.378) (end 207.264 103.378) (width 0.4) (layer "F.Cu") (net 2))
 (segment (start 207.264 103.378) (end 212.979 97.663) (width 0.4) (layer "F.Cu") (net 2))
 (segment (start 204.978 103.7855) (end 203.1175 103.7855) (width 0.4) (layer "F.Cu") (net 2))
 (segment (start 203.1175 103.7855) (end 203.03 103.698) (width 0.4) (layer "F.Cu") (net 2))
 (segment (start 205.3855 103.378) (end 204.978 103.7855) (width 0.4) (layer "F.Cu") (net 2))
 (segment (start 189.62 94.615) (end 188.37 94.615) (width 0.4) (layer "F.Cu") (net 10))
 (segment (start 187.452 91.313) (end 184.277 88.138) (width 0.4) (layer "F.Cu") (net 10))
 (segment (start 187.452 93.697) (end 187.452 91.313) (width 0.4) (layer "F.Cu") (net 10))
 (segment (start 188.37 94.615) (end 187.452 93.697) (width 0.4) (layer "F.Cu") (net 10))
 (segment (start 184.912 90.678) (end 184.277 90.678) (width 0.4) (layer "F.Cu") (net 11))
 (segment (start 188.37 95.885) (end 186.436 93.951) (width 0.4) (layer "F.Cu") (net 11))
 (segment (start 186.436 92.202) (end 184.912 90.678) (width 0.4) (layer "F.Cu") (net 11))
 (segment (start 189.62 95.885) (end 188.37 95.885) (width 0.4) (layer "F.Cu") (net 11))
 (segment (start 186.436 93.951) (end 186.436 92.202) (width 0.4) (layer "F.Cu") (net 11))
 (segment (start 210.82 91.44) (end 209.042 89.662) (width 0.4) (layer "F.Cu") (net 34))
 (segment (start 209.042 89.662) (end 209.042 88.651998) (width 0.4) (layer "F.Cu") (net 34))
 (segment (start 209.042 88.651998) (end 207.385002 86.995) (width 0.4) (layer "F.Cu") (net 34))
 (segment (start 207.385002 86.995) (end 206.62 86.995) (width 0.4) (layer "F.Cu") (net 34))
 (segment (start 207.645 99.695) (end 206.62 99.695) (width 0.4) (layer "F.Cu") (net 24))
 (segment (start 210.82 96.52) (end 207.645 99.695) (width 0.4) (layer "F.Cu") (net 24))
 (segment (start 198.8445 105.598) (end 198.7785 105.664) (width 0.4) (layer "F.Cu") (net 37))
 (segment (start 200.83 105.598) (end 198.8445 105.598) (width 0.4) (layer "F.Cu") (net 37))
 (segment (start 210.82 93.98) (end 210.82 93.726) (width 0.4) (layer "F.Cu") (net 33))
 (segment (start 208.28 91.186) (end 208.28 89.159998) (width 0.4) (layer "F.Cu") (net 33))
 (segment (start 207.385002 88.265) (end 206.62 88.265) (width 0.4) (layer "F.Cu") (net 33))
 (segment (start 210.82 93.726) (end 208.28 91.186) (width 0.4) (layer "F.Cu") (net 33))
 (segment (start 208.28 89.159998) (end 207.385002 88.265) (width 0.4) (layer "F.Cu") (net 33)))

